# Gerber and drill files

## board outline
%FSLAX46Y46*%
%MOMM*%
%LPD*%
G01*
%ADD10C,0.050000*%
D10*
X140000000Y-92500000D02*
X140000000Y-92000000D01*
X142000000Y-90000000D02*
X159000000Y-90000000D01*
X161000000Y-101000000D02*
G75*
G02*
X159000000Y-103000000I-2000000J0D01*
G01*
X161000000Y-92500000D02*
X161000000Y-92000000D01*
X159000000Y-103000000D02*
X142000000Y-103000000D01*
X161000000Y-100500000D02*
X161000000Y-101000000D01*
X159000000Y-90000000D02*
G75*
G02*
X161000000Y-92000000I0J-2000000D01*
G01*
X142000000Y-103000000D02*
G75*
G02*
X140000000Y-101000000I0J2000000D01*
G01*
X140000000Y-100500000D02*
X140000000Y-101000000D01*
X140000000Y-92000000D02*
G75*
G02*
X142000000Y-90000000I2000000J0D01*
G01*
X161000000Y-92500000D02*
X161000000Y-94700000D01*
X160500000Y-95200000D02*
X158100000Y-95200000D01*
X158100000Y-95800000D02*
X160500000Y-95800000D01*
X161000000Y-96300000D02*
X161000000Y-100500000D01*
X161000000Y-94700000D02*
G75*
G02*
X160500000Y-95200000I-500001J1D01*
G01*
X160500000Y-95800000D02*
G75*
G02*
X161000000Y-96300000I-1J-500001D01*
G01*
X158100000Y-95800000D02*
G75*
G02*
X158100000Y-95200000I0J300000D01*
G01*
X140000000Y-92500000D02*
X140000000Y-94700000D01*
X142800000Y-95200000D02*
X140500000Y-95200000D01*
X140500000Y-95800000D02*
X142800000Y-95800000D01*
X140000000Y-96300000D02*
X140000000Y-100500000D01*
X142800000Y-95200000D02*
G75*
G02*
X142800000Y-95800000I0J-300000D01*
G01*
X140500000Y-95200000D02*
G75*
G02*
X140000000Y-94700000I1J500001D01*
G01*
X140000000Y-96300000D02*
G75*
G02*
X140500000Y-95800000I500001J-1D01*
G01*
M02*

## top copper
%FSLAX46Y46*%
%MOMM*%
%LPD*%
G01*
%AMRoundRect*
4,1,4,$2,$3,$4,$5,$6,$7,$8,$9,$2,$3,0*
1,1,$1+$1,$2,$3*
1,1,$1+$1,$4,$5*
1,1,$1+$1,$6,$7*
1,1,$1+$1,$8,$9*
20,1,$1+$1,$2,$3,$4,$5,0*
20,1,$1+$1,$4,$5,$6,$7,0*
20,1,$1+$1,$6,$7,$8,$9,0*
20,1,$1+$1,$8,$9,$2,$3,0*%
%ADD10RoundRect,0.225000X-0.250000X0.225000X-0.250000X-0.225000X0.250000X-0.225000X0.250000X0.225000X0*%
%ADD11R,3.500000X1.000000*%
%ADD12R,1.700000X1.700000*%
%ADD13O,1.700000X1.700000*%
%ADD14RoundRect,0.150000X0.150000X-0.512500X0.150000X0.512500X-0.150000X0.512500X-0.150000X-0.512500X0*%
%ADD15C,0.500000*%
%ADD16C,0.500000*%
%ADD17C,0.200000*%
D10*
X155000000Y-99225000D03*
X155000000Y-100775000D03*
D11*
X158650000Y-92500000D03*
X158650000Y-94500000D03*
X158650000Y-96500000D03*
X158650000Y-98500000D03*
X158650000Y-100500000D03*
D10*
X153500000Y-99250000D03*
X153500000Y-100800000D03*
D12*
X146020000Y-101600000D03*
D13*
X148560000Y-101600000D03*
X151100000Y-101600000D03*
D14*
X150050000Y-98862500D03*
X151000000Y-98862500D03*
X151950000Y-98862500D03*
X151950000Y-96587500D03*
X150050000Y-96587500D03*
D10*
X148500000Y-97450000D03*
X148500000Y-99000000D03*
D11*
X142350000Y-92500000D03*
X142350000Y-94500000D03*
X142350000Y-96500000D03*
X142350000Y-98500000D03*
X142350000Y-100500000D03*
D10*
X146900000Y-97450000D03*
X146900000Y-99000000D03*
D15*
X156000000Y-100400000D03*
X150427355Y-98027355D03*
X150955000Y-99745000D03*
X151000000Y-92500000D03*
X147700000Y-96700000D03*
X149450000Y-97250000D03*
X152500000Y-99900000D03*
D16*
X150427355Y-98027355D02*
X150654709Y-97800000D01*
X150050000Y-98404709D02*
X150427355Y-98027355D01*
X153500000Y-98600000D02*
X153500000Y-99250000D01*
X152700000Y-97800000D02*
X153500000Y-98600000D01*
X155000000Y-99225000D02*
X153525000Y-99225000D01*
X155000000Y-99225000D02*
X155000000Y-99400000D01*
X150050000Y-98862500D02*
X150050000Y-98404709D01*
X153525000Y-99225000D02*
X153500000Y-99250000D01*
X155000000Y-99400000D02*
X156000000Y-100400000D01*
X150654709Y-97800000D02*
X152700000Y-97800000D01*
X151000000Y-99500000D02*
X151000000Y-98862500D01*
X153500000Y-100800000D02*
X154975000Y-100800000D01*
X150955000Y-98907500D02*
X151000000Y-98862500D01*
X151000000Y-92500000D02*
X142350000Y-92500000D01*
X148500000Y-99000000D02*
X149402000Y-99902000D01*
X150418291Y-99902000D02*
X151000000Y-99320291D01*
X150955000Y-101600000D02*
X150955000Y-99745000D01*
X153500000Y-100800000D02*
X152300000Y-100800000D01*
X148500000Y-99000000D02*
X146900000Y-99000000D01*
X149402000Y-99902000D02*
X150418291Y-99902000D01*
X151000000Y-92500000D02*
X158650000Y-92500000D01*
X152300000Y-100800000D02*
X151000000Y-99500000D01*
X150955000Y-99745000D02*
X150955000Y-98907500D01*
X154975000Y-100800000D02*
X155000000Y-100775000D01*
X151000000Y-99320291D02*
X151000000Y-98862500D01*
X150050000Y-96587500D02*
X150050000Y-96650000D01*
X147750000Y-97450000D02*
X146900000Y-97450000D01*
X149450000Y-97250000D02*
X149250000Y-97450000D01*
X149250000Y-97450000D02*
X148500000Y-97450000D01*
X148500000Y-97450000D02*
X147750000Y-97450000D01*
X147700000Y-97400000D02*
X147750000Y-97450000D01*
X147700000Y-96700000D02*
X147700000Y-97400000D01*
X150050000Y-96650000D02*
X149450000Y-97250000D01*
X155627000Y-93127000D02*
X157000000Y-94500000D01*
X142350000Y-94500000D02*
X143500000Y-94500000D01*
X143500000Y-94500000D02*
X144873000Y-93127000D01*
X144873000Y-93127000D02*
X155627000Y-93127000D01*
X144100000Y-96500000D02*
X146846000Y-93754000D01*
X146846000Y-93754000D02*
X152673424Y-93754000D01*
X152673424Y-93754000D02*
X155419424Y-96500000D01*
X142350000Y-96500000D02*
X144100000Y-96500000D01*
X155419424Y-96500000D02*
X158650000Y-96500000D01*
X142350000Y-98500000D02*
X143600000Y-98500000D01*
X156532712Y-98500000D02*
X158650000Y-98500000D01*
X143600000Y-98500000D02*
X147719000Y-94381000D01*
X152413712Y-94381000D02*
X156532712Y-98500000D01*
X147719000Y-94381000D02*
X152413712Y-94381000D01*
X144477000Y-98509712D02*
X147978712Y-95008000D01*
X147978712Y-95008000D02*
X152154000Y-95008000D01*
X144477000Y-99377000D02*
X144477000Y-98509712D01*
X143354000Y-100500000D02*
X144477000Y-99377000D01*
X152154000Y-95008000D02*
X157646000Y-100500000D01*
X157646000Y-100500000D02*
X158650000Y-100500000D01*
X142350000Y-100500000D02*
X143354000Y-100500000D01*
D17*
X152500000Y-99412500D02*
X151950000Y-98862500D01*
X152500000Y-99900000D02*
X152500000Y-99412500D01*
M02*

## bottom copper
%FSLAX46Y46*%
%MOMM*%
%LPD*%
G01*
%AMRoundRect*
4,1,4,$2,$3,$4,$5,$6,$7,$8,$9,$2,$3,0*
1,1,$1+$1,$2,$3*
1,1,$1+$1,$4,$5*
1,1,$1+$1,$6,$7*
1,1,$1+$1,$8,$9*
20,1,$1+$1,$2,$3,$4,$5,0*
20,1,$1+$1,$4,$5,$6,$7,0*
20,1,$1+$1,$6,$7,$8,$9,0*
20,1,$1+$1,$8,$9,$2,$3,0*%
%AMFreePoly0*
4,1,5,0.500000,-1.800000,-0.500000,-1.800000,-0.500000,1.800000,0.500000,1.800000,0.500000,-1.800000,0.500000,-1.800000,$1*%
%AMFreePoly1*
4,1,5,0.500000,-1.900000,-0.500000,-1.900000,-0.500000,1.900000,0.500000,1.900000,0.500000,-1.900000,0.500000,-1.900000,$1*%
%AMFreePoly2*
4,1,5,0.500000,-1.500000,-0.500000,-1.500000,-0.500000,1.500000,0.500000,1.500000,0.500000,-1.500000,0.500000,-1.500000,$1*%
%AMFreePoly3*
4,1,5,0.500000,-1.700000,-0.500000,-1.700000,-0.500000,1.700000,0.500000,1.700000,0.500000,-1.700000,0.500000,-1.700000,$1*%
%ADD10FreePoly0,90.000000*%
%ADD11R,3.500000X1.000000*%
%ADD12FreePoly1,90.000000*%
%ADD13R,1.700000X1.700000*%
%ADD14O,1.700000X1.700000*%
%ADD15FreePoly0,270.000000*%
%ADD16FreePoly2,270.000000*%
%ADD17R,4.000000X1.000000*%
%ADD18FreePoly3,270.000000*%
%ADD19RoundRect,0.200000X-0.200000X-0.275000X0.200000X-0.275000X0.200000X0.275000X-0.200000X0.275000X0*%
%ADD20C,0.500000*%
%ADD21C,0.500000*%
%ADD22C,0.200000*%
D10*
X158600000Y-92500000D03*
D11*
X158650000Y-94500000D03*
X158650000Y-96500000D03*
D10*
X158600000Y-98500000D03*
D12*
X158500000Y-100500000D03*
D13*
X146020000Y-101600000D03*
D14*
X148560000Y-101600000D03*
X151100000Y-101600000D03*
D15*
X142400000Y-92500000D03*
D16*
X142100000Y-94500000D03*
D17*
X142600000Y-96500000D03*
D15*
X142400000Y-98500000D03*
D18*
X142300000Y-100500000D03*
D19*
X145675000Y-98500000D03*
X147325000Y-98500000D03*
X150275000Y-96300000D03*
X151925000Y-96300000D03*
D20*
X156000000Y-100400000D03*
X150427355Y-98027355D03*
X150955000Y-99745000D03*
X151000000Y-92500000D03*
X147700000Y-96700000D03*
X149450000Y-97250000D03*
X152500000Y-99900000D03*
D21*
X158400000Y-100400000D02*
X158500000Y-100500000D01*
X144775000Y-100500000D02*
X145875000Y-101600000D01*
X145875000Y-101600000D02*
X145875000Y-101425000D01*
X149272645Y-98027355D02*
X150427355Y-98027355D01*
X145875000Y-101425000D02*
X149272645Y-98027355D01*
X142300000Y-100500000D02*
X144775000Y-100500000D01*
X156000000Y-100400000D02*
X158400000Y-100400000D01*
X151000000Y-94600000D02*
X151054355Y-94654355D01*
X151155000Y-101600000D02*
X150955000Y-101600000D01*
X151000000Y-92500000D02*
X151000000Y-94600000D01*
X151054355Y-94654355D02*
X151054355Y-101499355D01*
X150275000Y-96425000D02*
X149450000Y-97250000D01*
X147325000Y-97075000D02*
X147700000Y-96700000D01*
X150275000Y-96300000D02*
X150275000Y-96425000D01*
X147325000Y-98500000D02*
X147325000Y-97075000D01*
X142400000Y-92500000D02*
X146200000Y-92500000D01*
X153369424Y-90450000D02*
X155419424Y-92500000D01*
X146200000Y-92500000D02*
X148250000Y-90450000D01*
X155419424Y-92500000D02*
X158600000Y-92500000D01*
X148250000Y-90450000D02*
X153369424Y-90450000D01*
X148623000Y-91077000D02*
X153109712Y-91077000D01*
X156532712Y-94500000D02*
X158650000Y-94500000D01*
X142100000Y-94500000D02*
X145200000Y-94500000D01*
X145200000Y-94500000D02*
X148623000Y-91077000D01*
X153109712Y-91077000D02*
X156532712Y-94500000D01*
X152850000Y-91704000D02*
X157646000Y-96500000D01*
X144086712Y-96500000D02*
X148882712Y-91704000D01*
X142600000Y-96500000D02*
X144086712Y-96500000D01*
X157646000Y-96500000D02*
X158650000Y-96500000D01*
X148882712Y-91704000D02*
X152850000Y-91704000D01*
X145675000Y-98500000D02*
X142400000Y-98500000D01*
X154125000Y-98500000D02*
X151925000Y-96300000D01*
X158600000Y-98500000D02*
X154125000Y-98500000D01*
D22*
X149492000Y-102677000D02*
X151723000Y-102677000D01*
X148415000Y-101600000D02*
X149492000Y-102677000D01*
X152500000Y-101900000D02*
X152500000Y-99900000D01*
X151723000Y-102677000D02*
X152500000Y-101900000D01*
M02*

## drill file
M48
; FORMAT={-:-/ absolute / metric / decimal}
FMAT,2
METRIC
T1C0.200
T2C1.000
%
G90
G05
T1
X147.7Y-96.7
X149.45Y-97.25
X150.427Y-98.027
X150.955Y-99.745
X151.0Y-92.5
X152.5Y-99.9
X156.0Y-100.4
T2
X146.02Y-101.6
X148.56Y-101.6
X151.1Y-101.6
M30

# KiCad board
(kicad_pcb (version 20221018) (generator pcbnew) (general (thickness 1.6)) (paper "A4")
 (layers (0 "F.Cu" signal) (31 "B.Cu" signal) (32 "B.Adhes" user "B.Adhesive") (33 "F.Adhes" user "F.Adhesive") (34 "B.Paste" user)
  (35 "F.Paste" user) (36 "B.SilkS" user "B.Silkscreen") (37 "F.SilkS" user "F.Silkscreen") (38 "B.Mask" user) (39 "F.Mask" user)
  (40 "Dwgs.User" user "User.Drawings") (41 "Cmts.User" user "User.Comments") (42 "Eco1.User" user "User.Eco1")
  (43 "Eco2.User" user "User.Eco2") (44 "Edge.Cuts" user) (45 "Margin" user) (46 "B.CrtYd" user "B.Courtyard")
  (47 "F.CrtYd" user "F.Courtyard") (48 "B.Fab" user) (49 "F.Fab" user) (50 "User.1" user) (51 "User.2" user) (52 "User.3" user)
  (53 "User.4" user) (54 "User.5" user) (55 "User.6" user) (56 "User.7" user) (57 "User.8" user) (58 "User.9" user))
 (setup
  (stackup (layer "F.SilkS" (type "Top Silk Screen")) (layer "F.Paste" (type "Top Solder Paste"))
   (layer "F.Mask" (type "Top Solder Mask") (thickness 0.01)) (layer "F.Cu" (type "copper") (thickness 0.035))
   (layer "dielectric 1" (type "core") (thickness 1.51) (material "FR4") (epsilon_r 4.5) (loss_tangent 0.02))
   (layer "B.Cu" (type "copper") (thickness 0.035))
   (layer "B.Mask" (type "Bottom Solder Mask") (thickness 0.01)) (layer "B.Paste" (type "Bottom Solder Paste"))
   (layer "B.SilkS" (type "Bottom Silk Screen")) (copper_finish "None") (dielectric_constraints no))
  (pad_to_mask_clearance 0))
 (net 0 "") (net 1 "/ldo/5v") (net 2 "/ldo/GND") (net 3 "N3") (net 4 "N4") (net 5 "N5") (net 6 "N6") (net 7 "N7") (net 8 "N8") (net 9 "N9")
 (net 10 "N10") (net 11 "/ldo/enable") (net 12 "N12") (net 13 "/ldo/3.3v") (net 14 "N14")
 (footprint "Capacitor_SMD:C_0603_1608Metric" (layer "F.Cu") (at 155 100 -90)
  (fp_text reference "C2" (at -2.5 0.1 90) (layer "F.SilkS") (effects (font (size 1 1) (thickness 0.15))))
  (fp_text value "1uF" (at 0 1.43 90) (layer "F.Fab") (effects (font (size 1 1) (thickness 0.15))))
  (pad "1" smd roundrect (at -0.775 0 270) (size 0.9 0.95) (layers "F.Cu" "F.Paste" "F.Mask") (roundrect_rratio 0.25) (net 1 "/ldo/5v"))
  (pad "2" smd roundrect (at 0.775 0 270) (size 0.9 0.95) (layers "F.Cu" "F.Paste" "F.Mask") (roundrect_rratio 0.25) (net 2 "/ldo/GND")))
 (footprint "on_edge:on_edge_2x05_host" (layer "F.Cu") (at 161 96.5 -90)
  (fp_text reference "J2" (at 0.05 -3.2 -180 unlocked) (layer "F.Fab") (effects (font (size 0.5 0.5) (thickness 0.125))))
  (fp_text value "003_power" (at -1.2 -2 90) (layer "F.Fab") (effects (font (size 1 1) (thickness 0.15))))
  (fp_line (start -4 0) (end -1.8 0) (stroke (width 0.05) (type solid)) (layer "Edge.Cuts"))
  (fp_line (start -1.3 0.5) (end -1.3 2.9) (stroke (width 0.05) (type solid)) (layer "Edge.Cuts"))
  (fp_line (start -0.7 2.9) (end -0.7 0.5) (stroke (width 0.05) (type solid)) (layer "Edge.Cuts"))
  (fp_line (start -0.2 0) (end 4 0) (stroke (width 0.05) (type solid)) (layer "Edge.Cuts"))
  (fp_arc (start -1.8 0) (mid -1.446447 0.146447) (end -1.3 0.5) (stroke (width 0.05) (type solid)) (layer "Edge.Cuts"))
  (fp_arc (start -0.7 0.5) (mid -0.553553 0.146447) (end -0.2 0) (stroke (width 0.05) (type solid)) (layer "Edge.Cuts"))
  (fp_arc (start -0.7 2.9) (mid -1 3.2) (end -1.3 2.9) (stroke (width 0.05) (type solid)) (layer "Edge.Cuts"))
  (pad "1" smd rect (at -4 2.35 270) (size 1 3.5) (layers "F.Cu" "F.Mask") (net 2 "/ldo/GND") (zone_connect 0))
  (pad "2" smd rect (at -2 2.35 270) (size 1 3.5) (layers "F.Cu" "F.Mask") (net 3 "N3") (zone_connect 0))
  (pad "3" smd rect (at 0 2.35 270) (size 1 3.5) (layers "F.Cu" "F.Mask") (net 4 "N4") (zone_connect 0))
  (pad "4" smd rect (at 2 2.35 270) (size 1 3.5) (layers "F.Cu" "F.Mask") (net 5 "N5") (zone_connect 0))
  (pad "5" smd rect (at 4 2.35 270) (size 1 3.5) (layers "F.Cu" "F.Mask") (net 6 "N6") (zone_connect 0))
  (pad "6" smd custom (at -4 2.4 90) (size 1 3.6) (layers "B.Cu" "B.Mask") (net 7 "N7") (zone_connect 0) (thermal_bridge_angle 45)
   (options (clearance outline) (anchor rect)) (primitives))
  (pad "7" smd rect (at -2 2.35 90) (size 1 3.5) (layers "B.Cu" "B.Mask") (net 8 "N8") (zone_connect 0))
  (pad "8" smd rect (at 0 2.35 90) (size 1 3.5) (layers "B.Cu" "B.Mask") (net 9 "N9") (zone_connect 0))
  (pad "9" smd custom (at 2 2.4 90) (size 1 3.6) (layers "B.Cu" "B.Mask") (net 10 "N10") (zone_connect 0) (thermal_bridge_angle 45)
   (options (clearance outline) (anchor rect)) (primitives))
  (pad "10" smd custom (at 4 2.5 90) (size 1 3.8) (layers "B.Cu" "B.Mask") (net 1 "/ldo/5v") (zone_connect 0) (thermal_bridge_angle 45)
   (options (clearance outline) (anchor rect)) (primitives))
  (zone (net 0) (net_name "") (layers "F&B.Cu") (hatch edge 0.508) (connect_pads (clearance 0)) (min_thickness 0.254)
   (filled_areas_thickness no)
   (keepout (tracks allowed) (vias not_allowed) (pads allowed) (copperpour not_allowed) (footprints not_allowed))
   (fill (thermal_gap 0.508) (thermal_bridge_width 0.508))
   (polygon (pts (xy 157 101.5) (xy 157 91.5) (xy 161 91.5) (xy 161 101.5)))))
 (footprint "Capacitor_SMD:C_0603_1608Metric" (layer "F.Cu") (at 153.5 100.025 -90)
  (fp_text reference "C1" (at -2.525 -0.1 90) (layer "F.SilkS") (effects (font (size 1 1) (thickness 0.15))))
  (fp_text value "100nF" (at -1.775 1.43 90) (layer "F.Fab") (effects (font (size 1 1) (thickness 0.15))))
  (pad "1" smd roundrect (at -0.775 0 270) (size 0.9 0.95) (layers "F.Cu" "F.Paste" "F.Mask") (roundrect_rratio 0.25) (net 1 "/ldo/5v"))
  (pad "2" smd roundrect (at 0.775 0 270) (size 0.9 0.95) (layers "F.Cu" "F.Paste" "F.Mask") (roundrect_rratio 0.25) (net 2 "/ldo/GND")))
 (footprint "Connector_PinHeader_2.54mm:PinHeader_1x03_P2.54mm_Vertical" (layer "F.Cu") (at 146.02 101.6 90)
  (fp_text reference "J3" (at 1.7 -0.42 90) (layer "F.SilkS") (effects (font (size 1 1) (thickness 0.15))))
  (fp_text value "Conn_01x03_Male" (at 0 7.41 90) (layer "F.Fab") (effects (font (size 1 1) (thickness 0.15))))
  (pad "1" thru_hole rect (at 0 0 90) (size 1.7 1.7) (drill 1) (layers "*.Cu" "*.Mask") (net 1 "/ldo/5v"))
  (pad "2" thru_hole oval (at 0 2.54 90) (size 1.7 1.7) (drill 1) (layers "*.Cu" "*.Mask") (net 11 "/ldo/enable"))
  (pad "3" thru_hole oval (at 0 5.08 90) (size 1.7 1.7) (drill 1) (layers "*.Cu" "*.Mask") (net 2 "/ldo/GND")))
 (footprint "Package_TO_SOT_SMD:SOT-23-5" (layer "F.Cu") (at 151 97.725 90)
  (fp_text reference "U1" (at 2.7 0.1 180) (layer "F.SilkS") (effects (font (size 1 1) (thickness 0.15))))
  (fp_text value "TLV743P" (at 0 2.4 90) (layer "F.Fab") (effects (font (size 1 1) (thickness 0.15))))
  (pad "1" smd roundrect (at -1.1375 -0.95 90) (size 1.325 0.6) (layers "F.Cu" "F.Paste" "F.Mask") (roundrect_rratio 0.25) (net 1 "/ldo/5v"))
  (pad "2" smd roundrect (at -1.1375 0 90) (size 1.325 0.6) (layers "F.Cu" "F.Paste" "F.Mask") (roundrect_rratio 0.25) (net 2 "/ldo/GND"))
  (pad "3" smd roundrect (at -1.1375 0.95 90) (size 1.325 0.6) (layers "F.Cu" "F.Paste" "F.Mask") (roundrect_rratio 0.25)
   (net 11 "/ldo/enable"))
  (pad "4" smd roundrect (at 1.1375 0.95 90) (size 1.325 0.6) (layers "F.Cu" "F.Paste" "F.Mask") (roundrect_rratio 0.25) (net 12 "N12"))
  (pad "5" smd roundrect (at 1.1375 -0.95 90) (size 1.325 0.6) (layers "F.Cu" "F.Paste" "F.Mask") (roundrect_rratio 0.25)
   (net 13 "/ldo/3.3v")))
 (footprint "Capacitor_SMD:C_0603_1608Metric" (layer "F.Cu") (at 148.5 98.225 -90)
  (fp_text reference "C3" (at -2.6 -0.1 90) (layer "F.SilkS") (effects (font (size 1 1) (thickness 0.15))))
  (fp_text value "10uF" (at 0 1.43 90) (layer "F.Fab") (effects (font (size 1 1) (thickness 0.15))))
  (pad "1" smd roundrect (at -0.775 0 270) (size 0.9 0.95) (layers "F.Cu" "F.Paste" "F.Mask") (roundrect_rratio 0.25) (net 13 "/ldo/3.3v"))
  (pad "2" smd roundrect (at 0.775 0 270) (size 0.9 0.95) (layers "F.Cu" "F.Paste" "F.Mask") (roundrect_rratio 0.25) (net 2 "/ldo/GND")))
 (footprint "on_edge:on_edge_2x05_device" (layer "F.Cu") (at 140 96.5 -90)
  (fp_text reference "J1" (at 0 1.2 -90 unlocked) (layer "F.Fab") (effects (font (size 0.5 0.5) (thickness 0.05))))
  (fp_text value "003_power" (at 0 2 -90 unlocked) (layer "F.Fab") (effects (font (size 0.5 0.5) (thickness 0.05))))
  (fp_line (start -4 0) (end -1.8 0) (stroke (width 0.05) (type solid)) (layer "Edge.Cuts"))
  (fp_line (start -1.3 -2.8) (end -1.3 -0.5) (stroke (width 0.05) (type solid)) (layer "Edge.Cuts"))
  (fp_line (start -0.7 -0.5) (end -0.7 -2.8) (stroke (width 0.05) (type solid)) (layer "Edge.Cuts"))
  (fp_line (start -0.2 0) (end 4 0) (stroke (width 0.05) (type solid)) (layer "Edge.Cuts"))
  (fp_arc (start -1.3 -2.8) (mid -1 -3.1) (end -0.7 -2.8) (stroke (width 0.05) (type solid)) (layer "Edge.Cuts"))
  (fp_arc (start -1.3 -0.5) (mid -1.446447 -0.146447) (end -1.8 0) (stroke (width 0.05) (type solid)) (layer "Edge.Cuts"))
  (fp_arc (start -0.2 0) (mid -0.553553 -0.146447) (end -0.7 -0.5) (stroke (width 0.05) (type solid)) (layer "Edge.Cuts"))
  (pad "1" smd rect (at -4 -2.35 90) (size 1 3.5) (layers "F.Cu" "F.Mask") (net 2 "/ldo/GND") (zone_connect 0))
  (pad "2" smd rect (at -2 -2.35 270) (size 1 3.5) (layers "F.Cu" "F.Mask") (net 3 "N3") (zone_connect 0))
  (pad "3" smd rect (at 0 -2.35 270) (size 1 3.5) (layers "F.Cu" "F.Mask") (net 4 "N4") (zone_connect 0))
  (pad "4" smd rect (at 2 -2.35 90) (size 1 3.5) (layers "F.Cu" "F.Mask") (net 5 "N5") (zone_connect 0))
  (pad "5" smd rect (at 4 -2.35 90) (size 1 3.5) (layers "F.Cu" "F.Mask") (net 6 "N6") (zone_connect 0))
  (pad "6" smd custom (at -4 -2.4 270) (size 1 3.6) (layers "B.Cu" "B.Mask") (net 7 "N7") (zone_connect 0) (thermal_bridge_angle 45)
   (options (clearance outline) (anchor rect)) (primitives))
  (pad "7" smd custom (at -2 -2.1 270) (size 1 3) (layers "B.Cu" "B.Mask") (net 8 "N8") (zone_connect 0) (thermal_bridge_angle 45)
   (options (clearance outline) (anchor rect)) (primitives))
  (pad "8" smd rect (at 0 -2.6 270) (size 1 4) (layers "B.Cu" "B.Mask") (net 9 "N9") (zone_connect 0))
  (pad "9" smd custom (at 2 -2.4 270) (size 1 3.6) (layers "B.Cu" "B.Mask") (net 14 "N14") (zone_connect 0) (thermal_bridge_angle 45)
   (options (clearance outline) (anchor rect)) (primitives))
  (pad "10" smd custom (at 4 -2.3 270) (size 1 3.4) (layers "B.Cu" "B.Mask") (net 1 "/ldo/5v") (zone_connect 0) (thermal_bridge_angle 45)
   (options (clearance outline) (anchor rect)) (primitives))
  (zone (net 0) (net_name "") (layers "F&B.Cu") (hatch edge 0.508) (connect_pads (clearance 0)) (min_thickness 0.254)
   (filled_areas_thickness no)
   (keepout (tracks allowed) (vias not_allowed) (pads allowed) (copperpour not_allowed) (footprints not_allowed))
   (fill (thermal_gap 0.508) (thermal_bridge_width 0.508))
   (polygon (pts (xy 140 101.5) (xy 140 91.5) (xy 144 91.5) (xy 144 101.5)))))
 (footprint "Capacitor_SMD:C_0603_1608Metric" (layer "F.Cu") (at 146.9 98.225 -90)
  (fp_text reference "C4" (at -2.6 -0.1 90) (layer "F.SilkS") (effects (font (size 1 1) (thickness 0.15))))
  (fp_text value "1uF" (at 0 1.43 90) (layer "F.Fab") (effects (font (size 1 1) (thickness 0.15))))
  (pad "1" smd roundrect (at -0.775 0 270) (size 0.9 0.95) (layers "F.Cu" "F.Paste" "F.Mask") (roundrect_rratio 0.25) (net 13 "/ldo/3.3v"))
  (pad "2" smd roundrect (at 0.775 0 270) (size 0.9 0.95) (layers "F.Cu" "F.Paste" "F.Mask") (roundrect_rratio 0.25) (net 2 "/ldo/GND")))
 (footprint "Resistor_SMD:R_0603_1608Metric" (layer "B.Cu") (at 146.5 98.5)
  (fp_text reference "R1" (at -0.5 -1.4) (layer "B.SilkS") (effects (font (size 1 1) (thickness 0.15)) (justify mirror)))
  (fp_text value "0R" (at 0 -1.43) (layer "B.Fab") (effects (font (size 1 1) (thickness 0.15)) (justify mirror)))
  (pad "1" smd roundrect (at -0.825 0) (size 0.8 0.95) (layers "B.Cu" "B.Paste" "B.Mask") (roundrect_rratio 0.25) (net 14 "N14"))
  (pad "2" smd roundrect (at 0.825 0) (size 0.8 0.95) (layers "B.Cu" "B.Paste" "B.Mask") (roundrect_rratio 0.25) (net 13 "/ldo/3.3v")))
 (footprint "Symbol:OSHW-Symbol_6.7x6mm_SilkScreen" (layer "B.Cu") (at 150.8 93.1 180)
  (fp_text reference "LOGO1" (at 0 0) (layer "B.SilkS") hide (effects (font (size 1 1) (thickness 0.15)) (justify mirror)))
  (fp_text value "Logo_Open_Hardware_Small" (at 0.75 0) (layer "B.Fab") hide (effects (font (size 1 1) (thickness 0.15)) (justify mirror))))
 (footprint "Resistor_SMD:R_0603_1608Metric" (layer "B.Cu") (at 151.1 96.3)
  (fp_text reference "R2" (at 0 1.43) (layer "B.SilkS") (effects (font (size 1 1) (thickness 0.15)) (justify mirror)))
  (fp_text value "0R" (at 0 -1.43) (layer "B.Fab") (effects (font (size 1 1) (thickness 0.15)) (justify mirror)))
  (pad "1" smd roundrect (at -0.825 0) (size 0.8 0.95) (layers "B.Cu" "B.Paste" "B.Mask") (roundrect_rratio 0.25) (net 13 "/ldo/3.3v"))
  (pad "2" smd roundrect (at 0.825 0) (size 0.8 0.95) (layers "B.Cu" "B.Paste" "B.Mask") (roundrect_rratio 0.25) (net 10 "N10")))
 (gr_line (start 140 92.5) (end 140 92) (stroke (width 0.05) (type solid)) (layer "Edge.Cuts"))
 (gr_line (start 142 90) (end 159 90) (stroke (width 0.05) (type solid)) (layer "Edge.Cuts"))
 (gr_arc (start 161 101) (mid 160.414214 102.414214) (end 159 103) (stroke (width 0.05) (type solid)) (layer "Edge.Cuts"))
 (gr_line (start 161 92.5) (end 161 92) (stroke (width 0.05) (type solid)) (layer "Edge.Cuts"))
 (gr_line (start 159 103) (end 142 103) (stroke (width 0.05) (type solid)) (layer "Edge.Cuts"))
 (gr_line (start 161 100.5) (end 161 101) (stroke (width 0.05) (type solid)) (layer "Edge.Cuts"))
 (gr_arc (start 159 90) (mid 160.414214 90.585786) (end 161 92) (stroke (width 0.05) (type solid)) (layer "Edge.Cuts"))
 (gr_arc (start 142 103) (mid 140.585786 102.414214) (end 140 101) (stroke (width 0.05) (type solid)) (layer "Edge.Cuts"))
 (gr_line (start 140 100.5) (end 140 101) (stroke (width 0.05) (type solid)) (layer "Edge.Cuts"))
 (gr_arc (start 140 92) (mid 140.585786 90.585786) (end 142 90) (stroke (width 0.05) (type solid)) (layer "Edge.Cuts"))
 (segment (start 150.427355 98.027355) (end 150.654709 97.8) (width 0.5) (layer "F.Cu") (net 1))
 (segment (start 150.05 98.404709) (end 150.427355 98.027355) (width 0.5) (layer "F.Cu") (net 1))
 (segment (start 153.5 98.6) (end 153.5 99.25) (width 0.5) (layer "F.Cu") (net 1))
 (segment (start 152.7 97.8) (end 153.5 98.6) (width 0.5) (layer "F.Cu") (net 1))
 (segment (start 155 99.225) (end 153.525 99.225) (width 0.5) (layer "F.Cu") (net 1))
 (segment (start 155 99.225) (end 155 99.4) (width 0.5) (layer "F.Cu") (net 1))
 (segment (start 150.05 98.8625) (end 150.05 98.404709) (width 0.5) (layer "F.Cu") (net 1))
 (segment (start 153.525 99.225) (end 153.5 99.25) (width 0.5) (layer "F.Cu") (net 1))
 (segment (start 155 99.4) (end 156 100.4) (width 0.5) (layer "F.Cu") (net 1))
 (segment (start 150.654709 97.8) (end 152.7 97.8) (width 0.5) (layer "F.Cu") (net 1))
 (via (at 156 100.4) (size 0.5) (drill 0.2) (layers "F.Cu" "B.Cu") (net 1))
 (via (at 150.427355 98.027355) (size 0.5) (drill 0.2) (layers "F.Cu" "B.Cu") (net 1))
 (segment (start 158.4 100.4) (end 158.5 100.5) (width 0.5) (layer "B.Cu") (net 1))
 (segment (start 144.775 100.5) (end 145.875 101.6) (width 0.5) (layer "B.Cu") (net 1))
 (segment (start 145.875 101.6) (end 145.875 101.425) (width 0.5) (layer "B.Cu") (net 1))
 (segment (start 149.272645 98.027355) (end 150.427355 98.027355) (width 0.5) (layer "B.Cu") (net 1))
 (segment (start 145.875 101.425) (end 149.272645 98.027355) (width 0.5) (layer "B.Cu") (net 1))
 (segment (start 142.3 100.5) (end 144.775 100.5) (width 0.5) (layer "B.Cu") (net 1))
 (segment (start 156 100.4) (end 158.4 100.4) (width 0.5) (layer "B.Cu") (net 1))
 (segment (start 151 99.5) (end 151 98.8625) (width 0.5) (layer "F.Cu") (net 2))
 (segment (start 153.5 100.8) (end 154.975 100.8) (width 0.5) (layer "F.Cu") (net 2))
 (segment (start 150.955 98.9075) (end 151 98.8625) (width 0.5) (layer "F.Cu") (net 2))
 (segment (start 151 92.5) (end 142.35 92.5) (width 0.5) (layer "F.Cu") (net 2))
 (segment (start 148.5 99) (end 149.402 99.902) (width 0.5) (layer "F.Cu") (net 2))
 (segment (start 150.418291 99.902) (end 151 99.320291) (width 0.5) (layer "F.Cu") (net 2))
 (segment (start 150.955 101.6) (end 150.955 99.745) (width 0.5) (layer "F.Cu") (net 2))
 (segment (start 153.5 100.8) (end 152.3 100.8) (width 0.5) (layer "F.Cu") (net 2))
 (segment (start 148.5 99) (end 146.9 99) (width 0.5) (layer "F.Cu") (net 2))
 (segment (start 149.402 99.902) (end 150.418291 99.902) (width 0.5) (layer "F.Cu") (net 2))
 (segment (start 151 92.5) (end 158.65 92.5) (width 0.5) (layer "F.Cu") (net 2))
 (segment (start 152.3 100.8) (end 151 99.5) (width 0.5) (layer "F.Cu") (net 2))
 (segment (start 150.955 99.745) (end 150.955 98.9075) (width 0.5) (layer "F.Cu") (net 2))
 (segment (start 154.975 100.8) (end 155 100.775) (width 0.5) (layer "F.Cu") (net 2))
 (segment (start 151 99.320291) (end 151 98.8625) (width 0.5) (layer "F.Cu") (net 2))
 (via (at 150.955 99.745) (size 0.5) (drill 0.2) (layers "F.Cu" "B.Cu") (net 2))
 (via (at 151 92.5) (size 0.5) (drill 0.2) (layers "F.Cu" "B.Cu") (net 2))
 (segment (start 151 94.6) (end 151.054355 94.654355) (width 0.5) (layer "B.Cu") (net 2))
 (segment (start 151.155 101.6) (end 150.955 101.6) (width 0.5) (layer "B.Cu") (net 2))
 (segment (start 151 92.5) (end 151 94.6) (width 0.5) (layer "B.Cu") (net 2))
 (segment (start 151.054355 94.654355) (end 151.054355 101.499355) (width 0.5) (layer "B.Cu") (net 2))
 (segment (start 150.05 96.5875) (end 150.05 96.65) (width 0.5) (layer "F.Cu") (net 13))
 (segment (start 147.75 97.45) (end 146.9 97.45) (width 0.5) (layer "F.Cu") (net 13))
 (segment (start 149.45 97.25) (end 149.25 97.45) (width 0.5) (layer "F.Cu") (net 13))
 (segment (start 149.25 97.45) (end 148.5 97.45) (width 0.5) (layer "F.Cu") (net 13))
 (segment (start 148.5 97.45) (end 147.75 97.45) (width 0.5) (layer "F.Cu") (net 13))
 (segment (start 147.7 97.4) (end 147.75 97.45) (width 0.5) (layer "F.Cu") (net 13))
 (segment (start 147.7 96.7) (end 147.7 97.4) (width 0.5) (layer "F.Cu") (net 13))
 (segment (start 150.05 96.65) (end 149.45 97.25) (width 0.5) (layer "F.Cu") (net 13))
 (via (at 147.7 96.7) (size 0.5) (drill 0.2) (layers "F.Cu" "B.Cu") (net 13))
 (via (at 149.45 97.25) (size 0.5) (drill 0.2) (layers "F.Cu" "B.Cu") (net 13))
 (segment (start 150.275 96.425) (end 149.45 97.25) (width 0.5) (layer "B.Cu") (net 13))
 (segment (start 147.325 97.075) (end 147.7 96.7) (width 0.5) (layer "B.Cu") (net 13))
 (segment (start 150.275 96.3) (end 150.275 96.425) (width 0.5) (layer "B.Cu") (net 13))
 (segment (start 147.325 98.5) (end 147.325 97.075) (width 0.5) (layer "B.Cu") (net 13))
 (segment (start 155.627 93.127) (end 157 94.5) (width 0.5) (layer "F.Cu") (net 3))
 (segment (start 142.35 94.5) (end 143.5 94.5) (width 0.5) (layer "F.Cu") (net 3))
 (segment (start 143.5 94.5) (end 144.873 93.127) (width 0.5) (layer "F.Cu") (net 3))
 (segment (start 144.873 93.127) (end 155.627 93.127) (width 0.5) (layer "F.Cu") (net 3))
 (segment (start 144.1 96.5) (end 146.846 93.754) (width 0.5) (layer "F.Cu") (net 4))
 (segment (start 146.846 93.754) (end 152.673424 93.754) (width 0.5) (layer "F.Cu") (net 4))
 (segment (start 152.673424 93.754) (end 155.419424 96.5) (width 0.5) (layer "F.Cu") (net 4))
 (segment (start 142.35 96.5) (end 144.1 96.5) (width 0.5) (layer "F.Cu") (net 4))
 (segment (start 155.419424 96.5) (end 158.65 96.5) (width 0.5) (layer "F.Cu") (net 4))
 (segment (start 142.35 98.5) (end 143.6 98.5) (width 0.5) (layer "F.Cu") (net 5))
 (segment (start 156.532712 98.5) (end 158.65 98.5) (width 0.5) (layer "F.Cu") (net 5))
 (segment (start 143.6 98.5) (end 147.719 94.381) (width 0.5) (layer "F.Cu") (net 5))
 (segment (start 152.413712 94.381) (end 156.532712 98.5) (width 0.5) (layer "F.Cu") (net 5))
 (segment (start 147.719 94.381) (end 152.413712 94.381) (width 0.5) (layer "F.Cu") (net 5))
 (segment (start 144.477 98.509712) (end 147.978712 95.008) (width 0.5) (layer "F.Cu") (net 6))
 (segment (start 147.978712 95.008) (end 152.154 95.008) (width 0.5) (layer "F.Cu") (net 6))
 (segment (start 144.477 99.377) (end 144.477 98.509712) (width 0.5) (layer "F.Cu") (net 6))
 (segment (start 143.354 100.5) (end 144.477 99.377) (width 0.5) (layer "F.Cu") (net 6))
 (segment (start 152.154 95.008) (end 157.646 100.5) (width 0.5) (layer "F.Cu") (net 6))
 (segment (start 157.646 100.5) (end 158.65 100.5) (width 0.5) (layer "F.Cu") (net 6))
 (segment (start 142.35 100.5) (end 143.354 100.5) (width 0.5) (layer "F.Cu") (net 6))
 (segment (start 142.4 92.5) (end 146.2 92.5) (width 0.5) (layer "B.Cu") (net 7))
 (segment (start 153.369424 90.45) (end 155.419424 92.5) (width 0.5) (layer "B.Cu") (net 7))
 (segment (start 146.2 92.5) (end 148.25 90.45) (width 0.5) (layer "B.Cu") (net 7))
 (segment (start 155.419424 92.5) (end 158.6 92.5) (width 0.5) (layer "B.Cu") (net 7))
 (segment (start 148.25 90.45) (end 153.369424 90.45) (width 0.5) (layer "B.Cu") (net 7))
 (segment (start 148.623 91.077) (end 153.109712 91.077) (width 0.5) (layer "B.Cu") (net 8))
 (segment (start 156.532712 94.5) (end 158.65 94.5) (width 0.5) (layer "B.Cu") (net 8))
 (segment (start 142.1 94.5) (end 145.2 94.5) (width 0.5) (layer "B.Cu") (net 8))
 (segment (start 145.2 94.5) (end 148.623 91.077) (width 0.5) (layer "B.Cu") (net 8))
 (segment (start 153.109712 91.077) (end 156.532712 94.5) (width 0.5) (layer "B.Cu") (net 8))
 (segment (start 152.85 91.704) (end 157.646 96.5) (width 0.5) (layer "B.Cu") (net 9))
 (segment (start 144.086712 96.5) (end 148.882712 91.704) (width 0.5) (layer "B.Cu") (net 9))
 (segment (start 142.6 96.5) (end 144.086712 96.5) (width 0.5) (layer "B.Cu") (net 9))
 (segment (start 157.646 96.5) (end 158.65 96.5) (width 0.5) (layer "B.Cu") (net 9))
 (segment (start 148.882712 91.704) (end 152.85 91.704) (width 0.5) (layer "B.Cu") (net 9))
 (segment (start 145.675 98.5) (end 142.4 98.5) (width 0.5) (layer "B.Cu") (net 14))
 (segment (start 154.125 98.5) (end 151.925 96.3) (width 0.5) (layer "B.Cu") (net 10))
 (segment (start 158.6 98.5) (end 154.125 98.5) (width 0.5) (layer "B.Cu") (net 10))
 (segment (start 152.5 99.4125) (end 151.95 98.8625) (width 0.2) (layer "F.Cu") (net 11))
 (segment (start 152.5 99.9) (end 152.5 99.4125) (width 0.2) (layer "F.Cu") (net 11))
 (via (at 152.5 99.9) (size 0.5) (drill 0.2) (layers "F.Cu" "B.Cu") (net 11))
 (segment (start 149.492 102.677) (end 151.723 102.677) (width 0.2) (layer "B.Cu") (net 11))
 (segment (start 148.415 101.6) (end 149.492 102.677) (width 0.2) (layer "B.Cu") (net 11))
 (segment (start 152.5 101.9) (end 152.5 99.9) (width 0.2) (layer "B.Cu") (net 11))
 (segment (start 151.723 102.677) (end 152.5 101.9) (width 0.2) (layer "B.Cu") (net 11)))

